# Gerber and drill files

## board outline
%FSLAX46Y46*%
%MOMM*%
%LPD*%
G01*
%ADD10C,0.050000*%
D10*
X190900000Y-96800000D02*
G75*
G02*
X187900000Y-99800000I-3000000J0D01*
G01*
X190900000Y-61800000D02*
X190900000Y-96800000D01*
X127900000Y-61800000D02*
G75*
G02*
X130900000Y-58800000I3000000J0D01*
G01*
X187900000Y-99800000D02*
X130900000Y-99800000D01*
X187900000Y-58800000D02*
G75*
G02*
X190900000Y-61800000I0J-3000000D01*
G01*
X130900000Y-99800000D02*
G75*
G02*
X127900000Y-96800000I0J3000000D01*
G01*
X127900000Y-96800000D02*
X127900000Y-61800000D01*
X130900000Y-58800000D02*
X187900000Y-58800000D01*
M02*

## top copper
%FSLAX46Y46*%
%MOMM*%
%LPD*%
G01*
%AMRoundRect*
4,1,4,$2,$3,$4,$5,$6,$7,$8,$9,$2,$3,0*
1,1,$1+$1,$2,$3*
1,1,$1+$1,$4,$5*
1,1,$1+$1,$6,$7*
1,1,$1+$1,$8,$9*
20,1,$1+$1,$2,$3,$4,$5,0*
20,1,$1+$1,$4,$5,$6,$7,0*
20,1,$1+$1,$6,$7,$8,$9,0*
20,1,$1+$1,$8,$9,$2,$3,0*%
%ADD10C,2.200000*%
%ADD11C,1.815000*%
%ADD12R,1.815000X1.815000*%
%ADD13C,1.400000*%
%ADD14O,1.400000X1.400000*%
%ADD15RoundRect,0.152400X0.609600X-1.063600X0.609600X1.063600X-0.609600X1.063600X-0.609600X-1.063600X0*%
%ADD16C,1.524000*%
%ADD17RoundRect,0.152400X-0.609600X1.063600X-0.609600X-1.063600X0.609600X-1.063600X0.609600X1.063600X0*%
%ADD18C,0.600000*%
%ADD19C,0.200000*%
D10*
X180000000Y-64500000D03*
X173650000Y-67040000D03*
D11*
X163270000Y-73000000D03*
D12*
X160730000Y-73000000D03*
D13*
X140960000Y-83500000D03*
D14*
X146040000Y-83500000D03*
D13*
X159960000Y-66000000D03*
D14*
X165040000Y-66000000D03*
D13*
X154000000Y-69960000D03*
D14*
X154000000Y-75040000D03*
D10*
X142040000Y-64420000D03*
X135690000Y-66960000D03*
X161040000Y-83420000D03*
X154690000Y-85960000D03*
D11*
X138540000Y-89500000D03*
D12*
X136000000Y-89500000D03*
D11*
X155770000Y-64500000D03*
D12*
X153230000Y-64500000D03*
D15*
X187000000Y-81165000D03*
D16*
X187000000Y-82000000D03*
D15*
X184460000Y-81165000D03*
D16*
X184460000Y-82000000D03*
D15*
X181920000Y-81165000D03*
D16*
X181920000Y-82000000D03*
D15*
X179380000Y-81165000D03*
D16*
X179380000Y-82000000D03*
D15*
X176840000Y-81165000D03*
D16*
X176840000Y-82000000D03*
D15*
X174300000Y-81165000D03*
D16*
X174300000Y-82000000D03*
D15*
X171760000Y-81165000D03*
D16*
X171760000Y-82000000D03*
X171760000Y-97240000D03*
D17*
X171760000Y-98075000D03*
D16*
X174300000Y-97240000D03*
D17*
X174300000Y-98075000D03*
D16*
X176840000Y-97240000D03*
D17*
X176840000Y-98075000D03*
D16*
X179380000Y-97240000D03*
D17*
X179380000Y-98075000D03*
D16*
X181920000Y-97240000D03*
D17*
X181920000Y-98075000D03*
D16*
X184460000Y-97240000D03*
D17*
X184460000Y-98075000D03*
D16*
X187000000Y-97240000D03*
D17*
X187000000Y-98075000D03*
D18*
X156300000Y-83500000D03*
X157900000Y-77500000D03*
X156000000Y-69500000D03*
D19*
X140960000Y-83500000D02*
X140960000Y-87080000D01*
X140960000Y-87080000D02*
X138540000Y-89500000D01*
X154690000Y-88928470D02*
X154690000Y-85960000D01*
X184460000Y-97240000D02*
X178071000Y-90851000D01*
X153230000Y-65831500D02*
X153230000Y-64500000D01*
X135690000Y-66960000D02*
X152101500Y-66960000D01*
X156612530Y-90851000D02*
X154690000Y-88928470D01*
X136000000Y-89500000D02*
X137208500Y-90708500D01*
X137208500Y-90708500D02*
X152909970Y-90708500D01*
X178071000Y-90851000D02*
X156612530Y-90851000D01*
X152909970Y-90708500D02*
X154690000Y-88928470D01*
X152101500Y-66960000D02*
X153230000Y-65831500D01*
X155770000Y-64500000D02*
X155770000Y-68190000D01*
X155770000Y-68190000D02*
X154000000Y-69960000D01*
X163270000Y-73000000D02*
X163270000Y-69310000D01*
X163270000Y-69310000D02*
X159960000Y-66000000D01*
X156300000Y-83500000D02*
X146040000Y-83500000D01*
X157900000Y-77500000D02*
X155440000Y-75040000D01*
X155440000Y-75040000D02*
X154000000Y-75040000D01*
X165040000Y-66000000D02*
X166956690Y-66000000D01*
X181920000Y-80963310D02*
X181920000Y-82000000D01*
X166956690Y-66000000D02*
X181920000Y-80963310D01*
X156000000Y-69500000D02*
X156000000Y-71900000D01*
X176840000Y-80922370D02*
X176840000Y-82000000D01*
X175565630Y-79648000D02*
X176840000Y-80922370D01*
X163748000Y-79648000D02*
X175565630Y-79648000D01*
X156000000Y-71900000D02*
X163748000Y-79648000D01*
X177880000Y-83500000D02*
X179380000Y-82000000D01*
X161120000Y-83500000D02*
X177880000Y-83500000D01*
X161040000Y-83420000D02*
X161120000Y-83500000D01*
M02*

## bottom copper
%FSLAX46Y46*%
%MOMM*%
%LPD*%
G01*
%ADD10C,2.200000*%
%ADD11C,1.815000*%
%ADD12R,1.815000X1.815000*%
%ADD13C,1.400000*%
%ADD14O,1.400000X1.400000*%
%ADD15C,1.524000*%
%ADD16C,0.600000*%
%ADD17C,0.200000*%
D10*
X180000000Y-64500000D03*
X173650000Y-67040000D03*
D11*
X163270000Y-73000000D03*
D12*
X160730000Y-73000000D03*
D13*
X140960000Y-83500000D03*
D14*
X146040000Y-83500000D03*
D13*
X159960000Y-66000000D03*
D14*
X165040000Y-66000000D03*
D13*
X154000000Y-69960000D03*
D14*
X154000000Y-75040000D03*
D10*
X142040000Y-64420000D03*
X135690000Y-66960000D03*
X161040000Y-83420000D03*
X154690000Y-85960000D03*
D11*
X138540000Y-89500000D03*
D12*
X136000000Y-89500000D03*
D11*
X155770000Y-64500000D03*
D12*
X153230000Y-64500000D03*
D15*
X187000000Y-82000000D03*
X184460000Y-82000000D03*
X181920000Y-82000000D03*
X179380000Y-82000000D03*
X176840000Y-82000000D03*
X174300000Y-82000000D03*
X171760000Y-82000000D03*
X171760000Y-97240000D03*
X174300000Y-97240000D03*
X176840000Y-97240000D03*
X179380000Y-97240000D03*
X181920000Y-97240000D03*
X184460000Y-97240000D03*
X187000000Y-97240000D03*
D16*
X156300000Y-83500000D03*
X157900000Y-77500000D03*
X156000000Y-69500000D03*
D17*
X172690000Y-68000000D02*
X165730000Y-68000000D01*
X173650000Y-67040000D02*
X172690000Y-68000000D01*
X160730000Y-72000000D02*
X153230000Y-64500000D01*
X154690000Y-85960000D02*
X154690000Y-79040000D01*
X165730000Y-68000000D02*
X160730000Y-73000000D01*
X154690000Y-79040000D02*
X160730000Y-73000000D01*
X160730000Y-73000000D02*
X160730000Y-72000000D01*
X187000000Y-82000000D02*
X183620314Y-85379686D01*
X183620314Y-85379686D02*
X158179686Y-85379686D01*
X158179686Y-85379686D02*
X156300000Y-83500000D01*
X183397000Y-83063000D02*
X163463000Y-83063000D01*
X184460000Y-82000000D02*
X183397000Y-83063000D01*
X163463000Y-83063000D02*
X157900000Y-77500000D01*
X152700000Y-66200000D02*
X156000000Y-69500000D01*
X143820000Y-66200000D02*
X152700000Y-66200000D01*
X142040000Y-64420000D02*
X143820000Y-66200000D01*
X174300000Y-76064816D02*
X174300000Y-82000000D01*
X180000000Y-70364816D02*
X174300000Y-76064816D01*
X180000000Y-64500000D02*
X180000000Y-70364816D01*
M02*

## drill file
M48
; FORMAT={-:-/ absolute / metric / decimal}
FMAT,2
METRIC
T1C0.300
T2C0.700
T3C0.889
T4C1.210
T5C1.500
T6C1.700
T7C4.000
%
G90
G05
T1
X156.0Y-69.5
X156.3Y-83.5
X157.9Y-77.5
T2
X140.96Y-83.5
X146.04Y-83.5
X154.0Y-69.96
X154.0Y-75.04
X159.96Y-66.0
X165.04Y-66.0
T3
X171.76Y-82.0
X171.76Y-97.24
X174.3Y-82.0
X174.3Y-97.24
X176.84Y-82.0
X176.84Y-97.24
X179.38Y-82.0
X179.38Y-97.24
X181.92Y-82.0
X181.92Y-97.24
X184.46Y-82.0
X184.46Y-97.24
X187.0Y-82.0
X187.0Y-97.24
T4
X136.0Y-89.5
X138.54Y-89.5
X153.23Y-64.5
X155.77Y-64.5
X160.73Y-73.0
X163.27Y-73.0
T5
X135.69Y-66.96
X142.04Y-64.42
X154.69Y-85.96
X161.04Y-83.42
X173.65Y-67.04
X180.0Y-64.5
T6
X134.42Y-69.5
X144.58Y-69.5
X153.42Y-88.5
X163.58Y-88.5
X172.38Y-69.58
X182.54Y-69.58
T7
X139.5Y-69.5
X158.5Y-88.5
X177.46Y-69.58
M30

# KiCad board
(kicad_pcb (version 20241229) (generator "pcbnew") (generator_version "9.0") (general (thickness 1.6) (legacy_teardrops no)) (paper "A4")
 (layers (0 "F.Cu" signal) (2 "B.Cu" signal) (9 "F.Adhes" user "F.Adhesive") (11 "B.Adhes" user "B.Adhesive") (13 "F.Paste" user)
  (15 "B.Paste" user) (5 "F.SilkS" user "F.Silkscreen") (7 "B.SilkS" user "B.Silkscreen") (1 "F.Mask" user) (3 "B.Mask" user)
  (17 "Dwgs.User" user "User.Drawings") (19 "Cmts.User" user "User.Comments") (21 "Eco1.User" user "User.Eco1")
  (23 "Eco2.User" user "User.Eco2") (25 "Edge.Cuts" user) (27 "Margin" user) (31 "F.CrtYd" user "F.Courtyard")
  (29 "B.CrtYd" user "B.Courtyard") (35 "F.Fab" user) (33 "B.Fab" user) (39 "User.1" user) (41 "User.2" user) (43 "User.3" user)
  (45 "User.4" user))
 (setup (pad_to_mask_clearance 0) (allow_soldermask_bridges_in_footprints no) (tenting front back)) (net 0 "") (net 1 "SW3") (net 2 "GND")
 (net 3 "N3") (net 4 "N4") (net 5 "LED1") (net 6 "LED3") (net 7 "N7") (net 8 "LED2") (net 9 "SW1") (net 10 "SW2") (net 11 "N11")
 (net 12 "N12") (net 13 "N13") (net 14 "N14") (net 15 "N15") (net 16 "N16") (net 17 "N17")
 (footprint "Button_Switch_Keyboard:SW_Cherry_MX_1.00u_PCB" (layer "F.Cu") (at 180 64.5)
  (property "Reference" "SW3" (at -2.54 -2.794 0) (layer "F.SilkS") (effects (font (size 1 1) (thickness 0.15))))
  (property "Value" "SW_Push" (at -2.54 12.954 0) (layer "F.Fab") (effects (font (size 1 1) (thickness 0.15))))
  (pad "" np_thru_hole circle (at -7.62 5.08) (size 1.7 1.7) (drill 1.7) (layers "*.Cu" "*.Mask"))
  (pad "" np_thru_hole circle (at -2.54 5.08) (size 4 4) (drill 4) (layers "*.Cu" "*.Mask"))
  (pad "" np_thru_hole circle (at 2.54 5.08) (size 1.7 1.7) (drill 1.7) (layers "*.Cu" "*.Mask"))
  (pad "1" thru_hole circle (at 0 0) (size 2.2 2.2) (drill 1.5) (layers "*.Cu" "*.Mask") (remove_unused_layers no) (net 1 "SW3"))
  (pad "2" thru_hole circle (at -6.35 2.54) (size 2.2 2.2) (drill 1.5) (layers "*.Cu" "*.Mask") (remove_unused_layers no) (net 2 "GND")))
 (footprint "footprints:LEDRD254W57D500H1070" (layer "F.Cu") (at 162 73)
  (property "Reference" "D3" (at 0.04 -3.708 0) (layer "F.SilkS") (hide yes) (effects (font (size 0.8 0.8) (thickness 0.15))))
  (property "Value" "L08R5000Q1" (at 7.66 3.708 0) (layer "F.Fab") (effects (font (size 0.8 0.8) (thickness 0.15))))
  (pad "A" thru_hole circle (at 1.27 0) (size 1.815 1.815) (drill 1.21) (layers "*.Cu" "*.Mask") (remove_unused_layers no) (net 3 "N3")
   (solder_mask_margin 0.102))
  (pad "C" thru_hole rect (at -1.27 0) (size 1.815 1.815) (drill 1.21) (layers "*.Cu" "*.Mask") (remove_unused_layers no) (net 2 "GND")
   (solder_mask_margin 0.102)))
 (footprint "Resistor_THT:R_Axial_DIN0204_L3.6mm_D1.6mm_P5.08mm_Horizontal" (layer "F.Cu") (at 140.96 83.5)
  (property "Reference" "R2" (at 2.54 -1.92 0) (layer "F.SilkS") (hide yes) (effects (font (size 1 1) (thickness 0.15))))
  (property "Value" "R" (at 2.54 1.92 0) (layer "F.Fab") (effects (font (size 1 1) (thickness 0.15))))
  (pad "1" thru_hole circle (at 0 0) (size 1.4 1.4) (drill 0.7) (layers "*.Cu" "*.Mask") (remove_unused_layers no) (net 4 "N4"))
  (pad "2" thru_hole oval (at 5.08 0) (size 1.4 1.4) (drill 0.7) (layers "*.Cu" "*.Mask") (remove_unused_layers no) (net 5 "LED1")))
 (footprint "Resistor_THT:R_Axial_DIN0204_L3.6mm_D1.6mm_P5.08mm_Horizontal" (layer "F.Cu") (at 159.96 66)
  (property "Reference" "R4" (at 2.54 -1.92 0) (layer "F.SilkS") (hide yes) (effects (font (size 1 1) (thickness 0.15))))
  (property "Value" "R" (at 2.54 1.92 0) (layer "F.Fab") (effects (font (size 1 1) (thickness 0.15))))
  (pad "1" thru_hole circle (at 0 0) (size 1.4 1.4) (drill 0.7) (layers "*.Cu" "*.Mask") (remove_unused_layers no) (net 3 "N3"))
  (pad "2" thru_hole oval (at 5.08 0) (size 1.4 1.4) (drill 0.7) (layers "*.Cu" "*.Mask") (remove_unused_layers no) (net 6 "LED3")))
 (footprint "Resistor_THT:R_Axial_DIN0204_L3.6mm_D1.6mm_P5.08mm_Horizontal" (layer "F.Cu") (at 154 69.96 -90)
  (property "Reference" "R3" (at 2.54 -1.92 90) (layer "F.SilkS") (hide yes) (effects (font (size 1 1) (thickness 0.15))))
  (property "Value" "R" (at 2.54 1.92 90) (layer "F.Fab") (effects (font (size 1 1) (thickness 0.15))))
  (pad "1" thru_hole circle (at 0 0 270) (size 1.4 1.4) (drill 0.7) (layers "*.Cu" "*.Mask") (remove_unused_layers no) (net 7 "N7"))
  (pad "2" thru_hole oval (at 5.08 0 270) (size 1.4 1.4) (drill 0.7) (layers "*.Cu" "*.Mask") (remove_unused_layers no) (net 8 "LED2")))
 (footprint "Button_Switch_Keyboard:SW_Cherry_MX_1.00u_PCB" (layer "F.Cu") (at 142.04 64.42)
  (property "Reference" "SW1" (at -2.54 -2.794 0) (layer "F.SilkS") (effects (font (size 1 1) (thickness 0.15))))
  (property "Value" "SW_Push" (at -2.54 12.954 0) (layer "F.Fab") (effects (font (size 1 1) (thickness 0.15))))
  (pad "" np_thru_hole circle (at -7.62 5.08) (size 1.7 1.7) (drill 1.7) (layers "*.Cu" "*.Mask"))
  (pad "" np_thru_hole circle (at -2.54 5.08) (size 4 4) (drill 4) (layers "*.Cu" "*.Mask"))
  (pad "" np_thru_hole circle (at 2.54 5.08) (size 1.7 1.7) (drill 1.7) (layers "*.Cu" "*.Mask"))
  (pad "1" thru_hole circle (at 0 0) (size 2.2 2.2) (drill 1.5) (layers "*.Cu" "*.Mask") (remove_unused_layers no) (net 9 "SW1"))
  (pad "2" thru_hole circle (at -6.35 2.54) (size 2.2 2.2) (drill 1.5) (layers "*.Cu" "*.Mask") (remove_unused_layers no) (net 2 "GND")))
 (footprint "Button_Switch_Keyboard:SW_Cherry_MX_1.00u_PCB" (layer "F.Cu") (at 161.04 83.42)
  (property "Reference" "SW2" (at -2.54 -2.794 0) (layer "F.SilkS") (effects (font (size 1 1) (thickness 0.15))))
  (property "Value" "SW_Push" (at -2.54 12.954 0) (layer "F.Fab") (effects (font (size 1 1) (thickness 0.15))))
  (pad "" np_thru_hole circle (at -7.62 5.08) (size 1.7 1.7) (drill 1.7) (layers "*.Cu" "*.Mask"))
  (pad "" np_thru_hole circle (at -2.54 5.08) (size 4 4) (drill 4) (layers "*.Cu" "*.Mask"))
  (pad "" np_thru_hole circle (at 2.54 5.08) (size 1.7 1.7) (drill 1.7) (layers "*.Cu" "*.Mask"))
  (pad "1" thru_hole circle (at 0 0) (size 2.2 2.2) (drill 1.5) (layers "*.Cu" "*.Mask") (remove_unused_layers no) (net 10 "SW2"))
  (pad "2" thru_hole circle (at -6.35 2.54) (size 2.2 2.2) (drill 1.5) (layers "*.Cu" "*.Mask") (remove_unused_layers no) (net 2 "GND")))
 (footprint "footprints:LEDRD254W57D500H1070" (layer "F.Cu") (at 137.27 89.5)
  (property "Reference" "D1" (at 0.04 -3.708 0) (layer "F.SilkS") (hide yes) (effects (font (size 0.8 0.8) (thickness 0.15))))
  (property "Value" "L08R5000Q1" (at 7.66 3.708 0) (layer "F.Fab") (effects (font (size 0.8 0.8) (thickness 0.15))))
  (pad "A" thru_hole circle (at 1.27 0) (size 1.815 1.815) (drill 1.21) (layers "*.Cu" "*.Mask") (remove_unused_layers no) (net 4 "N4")
   (solder_mask_margin 0.102))
  (pad "C" thru_hole rect (at -1.27 0) (size 1.815 1.815) (drill 1.21) (layers "*.Cu" "*.Mask") (remove_unused_layers no) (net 2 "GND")
   (solder_mask_margin 0.102)))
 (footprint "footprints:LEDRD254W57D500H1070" (layer "F.Cu") (at 154.5 64.5)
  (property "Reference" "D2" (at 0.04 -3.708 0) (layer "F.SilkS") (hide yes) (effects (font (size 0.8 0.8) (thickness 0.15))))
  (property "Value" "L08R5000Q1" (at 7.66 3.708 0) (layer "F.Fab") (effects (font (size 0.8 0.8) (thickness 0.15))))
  (pad "A" thru_hole circle (at 1.27 0) (size 1.815 1.815) (drill 1.21) (layers "*.Cu" "*.Mask") (remove_unused_layers no) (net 7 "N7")
   (solder_mask_margin 0.102))
  (pad "C" thru_hole rect (at -1.27 0) (size 1.815 1.815) (drill 1.21) (layers "*.Cu" "*.Mask") (remove_unused_layers no) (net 2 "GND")
   (solder_mask_margin 0.102)))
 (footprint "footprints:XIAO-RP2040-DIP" (layer "F.Cu") (at 179.38 89.62 -90)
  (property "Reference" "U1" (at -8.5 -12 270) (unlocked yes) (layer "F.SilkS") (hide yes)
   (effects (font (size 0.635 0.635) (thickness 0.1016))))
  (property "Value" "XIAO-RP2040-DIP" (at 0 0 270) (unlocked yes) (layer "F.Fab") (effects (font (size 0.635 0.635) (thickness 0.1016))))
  (pad "1" smd roundrect (at -8.455 -7.62 90) (size 2.432 1.524) (layers "F.Cu" "F.Mask") (roundrect_rratio 0.1) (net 5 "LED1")
   (thermal_bridge_angle 45))
  (pad "1" thru_hole circle (at -7.62 -7.62 90) (size 1.524 1.524) (drill 0.889) (layers "*.Cu" "*.Mask") (remove_unused_layers no)
   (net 5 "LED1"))
  (pad "2" smd roundrect (at -8.455 -5.08 90) (size 2.432 1.524) (layers "F.Cu" "F.Mask") (roundrect_rratio 0.1) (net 8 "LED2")
   (thermal_bridge_angle 45))
  (pad "2" thru_hole circle (at -7.62 -5.08 90) (size 1.524 1.524) (drill 0.889) (layers "*.Cu" "*.Mask") (remove_unused_layers no)
   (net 8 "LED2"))
  (pad "3" smd roundrect (at -8.455 -2.54 90) (size 2.432 1.524) (layers "F.Cu" "F.Mask") (roundrect_rratio 0.1) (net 6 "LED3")
   (thermal_bridge_angle 45))
  (pad "3" thru_hole circle (at -7.62 -2.54 90) (size 1.524 1.524) (drill 0.889) (layers "*.Cu" "*.Mask") (remove_unused_layers no)
   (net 6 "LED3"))
  (pad "4" smd roundrect (at -8.455 0 90) (size 2.432 1.524) (layers "F.Cu" "F.Mask") (roundrect_rratio 0.1) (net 10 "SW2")
   (thermal_bridge_angle 45))
  (pad "4" thru_hole circle (at -7.62 0 90) (size 1.524 1.524) (drill 0.889) (layers "*.Cu" "*.Mask") (remove_unused_layers no)
   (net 10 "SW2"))
  (pad "5" smd roundrect (at -8.455 2.54 90) (size 2.432 1.524) (layers "F.Cu" "F.Mask") (roundrect_rratio 0.1) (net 9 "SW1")
   (thermal_bridge_angle 45))
  (pad "5" thru_hole circle (at -7.62 2.54 90) (size 1.524 1.524) (drill 0.889) (layers "*.Cu" "*.Mask") (remove_unused_layers no)
   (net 9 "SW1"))
  (pad "6" smd roundrect (at -8.455 5.08 90) (size 2.432 1.524) (layers "F.Cu" "F.Mask") (roundrect_rratio 0.1) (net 1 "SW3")
   (thermal_bridge_angle 45))
  (pad "6" thru_hole circle (at -7.62 5.08 90) (size 1.524 1.524) (drill 0.889) (layers "*.Cu" "*.Mask") (remove_unused_layers no)
   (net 1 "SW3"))
  (pad "7" smd roundrect (at -8.455 7.62 90) (size 2.432 1.524) (layers "F.Cu" "F.Mask") (roundrect_rratio 0.1) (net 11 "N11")
   (thermal_bridge_angle 45))
  (pad "7" thru_hole circle (at -7.62 7.62 90) (size 1.524 1.524) (drill 0.889) (layers "*.Cu" "*.Mask") (remove_unused_layers no)
   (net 11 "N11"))
  (pad "8" thru_hole circle (at 7.62 7.62 270) (size 1.524 1.524) (drill 0.889) (layers "*.Cu" "*.Mask") (remove_unused_layers no)
   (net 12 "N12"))
  (pad "8" smd roundrect (at 8.455 7.62 270) (size 2.432 1.524) (layers "F.Cu" "F.Mask") (roundrect_rratio 0.1) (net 12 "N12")
   (thermal_bridge_angle 45))
  (pad "9" thru_hole circle (at 7.62 5.08 270) (size 1.524 1.524) (drill 0.889) (layers "*.Cu" "*.Mask") (remove_unused_layers no)
   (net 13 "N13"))
  (pad "9" smd roundrect (at 8.455 5.08 270) (size 2.432 1.524) (layers "F.Cu" "F.Mask") (roundrect_rratio 0.1) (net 13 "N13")
   (thermal_bridge_angle 45))
  (pad "10" thru_hole circle (at 7.62 2.54 270) (size 1.524 1.524) (drill 0.889) (layers "*.Cu" "*.Mask") (remove_unused_layers no)
   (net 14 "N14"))
  (pad "10" smd roundrect (at 8.455 2.54 270) (size 2.432 1.524) (layers "F.Cu" "F.Mask") (roundrect_rratio 0.1) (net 14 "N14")
   (thermal_bridge_angle 45))
  (pad "11" thru_hole circle (at 7.62 0 270) (size 1.524 1.524) (drill 0.889) (layers "*.Cu" "*.Mask") (remove_unused_layers no)
   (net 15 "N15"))
  (pad "11" smd roundrect (at 8.455 0 270) (size 2.432 1.524) (layers "F.Cu" "F.Mask") (roundrect_rratio 0.1) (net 15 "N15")
   (thermal_bridge_angle 45))
  (pad "12" thru_hole circle (at 7.62 -2.54 270) (size 1.524 1.524) (drill 0.889) (layers "*.Cu" "*.Mask") (remove_unused_layers no)
   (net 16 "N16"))
  (pad "12" smd roundrect (at 8.455 -2.54 270) (size 2.432 1.524) (layers "F.Cu" "F.Mask") (roundrect_rratio 0.1) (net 16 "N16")
   (thermal_bridge_angle 45))
  (pad "13" thru_hole circle (at 7.62 -5.08 270) (size 1.524 1.524) (drill 0.889) (layers "*.Cu" "*.Mask") (remove_unused_layers no)
   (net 2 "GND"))
  (pad "13" smd roundrect (at 8.455 -5.08 270) (size 2.432 1.524) (layers "F.Cu" "F.Mask") (roundrect_rratio 0.1) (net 2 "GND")
   (thermal_bridge_angle 45))
  (pad "14" thru_hole circle (at 7.62 -7.62 270) (size 1.524 1.524) (drill 0.889) (layers "*.Cu" "*.Mask") (remove_unused_layers no)
   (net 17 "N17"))
  (pad "14" smd roundrect (at 8.455 -7.62 270) (size 2.432 1.524) (layers "F.Cu" "F.Mask") (roundrect_rratio 0.1) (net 17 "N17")
   (thermal_bridge_angle 45)))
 (gr_arc (start 190.9 96.8) (mid 190.02132 98.92132) (end 187.9 99.8) (stroke (width 0.05) (type default)) (layer "Edge.Cuts"))
 (gr_line (start 190.9 61.8) (end 190.9 96.8) (stroke (width 0.05) (type default)) (layer "Edge.Cuts"))
 (gr_arc (start 127.9 61.8) (mid 128.77868 59.67868) (end 130.9 58.8) (stroke (width 0.05) (type default)) (layer "Edge.Cuts"))
 (gr_line (start 187.9 99.8) (end 130.9 99.8) (stroke (width 0.05) (type default)) (layer "Edge.Cuts"))
 (gr_arc (start 187.9 58.8) (mid 190.02132 59.67868) (end 190.9 61.8) (stroke (width 0.05) (type default)) (layer "Edge.Cuts"))
 (gr_arc (start 130.9 99.8) (mid 128.77868 98.92132) (end 127.9 96.8) (stroke (width 0.05) (type default)) (layer "Edge.Cuts"))
 (gr_line (start 127.9 96.8) (end 127.9 61.8) (stroke (width 0.05) (type default)) (layer "Edge.Cuts"))
 (gr_line (start 130.9 58.8) (end 187.9 58.8) (stroke (width 0.05) (type default)) (layer "Edge.Cuts"))
 (segment (start 140.96 83.5) (end 140.96 87.08) (width 0.2) (layer "F.Cu") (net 4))
 (segment (start 140.96 87.08) (end 138.54 89.5) (width 0.2) (layer "F.Cu") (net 4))
 (segment (start 154.69 88.92847) (end 154.69 85.96) (width 0.2) (layer "F.Cu") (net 2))
 (segment (start 184.46 97.24) (end 178.071 90.851) (width 0.2) (layer "F.Cu") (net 2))
 (segment (start 153.23 65.8315) (end 153.23 64.5) (width 0.2) (layer "F.Cu") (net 2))
 (segment (start 135.69 66.96) (end 152.1015 66.96) (width 0.2) (layer "F.Cu") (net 2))
 (segment (start 156.61253 90.851) (end 154.69 88.92847) (width 0.2) (layer "F.Cu") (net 2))
 (segment (start 136 89.5) (end 137.2085 90.7085) (width 0.2) (layer "F.Cu") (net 2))
 (segment (start 137.2085 90.7085) (end 152.90997 90.7085) (width 0.2) (layer "F.Cu") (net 2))
 (segment (start 178.071 90.851) (end 156.61253 90.851) (width 0.2) (layer "F.Cu") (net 2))
 (segment (start 152.90997 90.7085) (end 154.69 88.92847) (width 0.2) (layer "F.Cu") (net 2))
 (segment (start 152.1015 66.96) (end 153.23 65.8315) (width 0.2) (layer "F.Cu") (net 2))
 (segment (start 172.69 68) (end 165.73 68) (width 0.2) (layer "B.Cu") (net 2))
 (segment (start 173.65 67.04) (end 172.69 68) (width 0.2) (layer "B.Cu") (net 2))
 (segment (start 160.73 72) (end 153.23 64.5) (width 0.2) (layer "B.Cu") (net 2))
 (segment (start 154.69 85.96) (end 154.69 79.04) (width 0.2) (layer "B.Cu") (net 2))
 (segment (start 165.73 68) (end 160.73 73) (width 0.2) (layer "B.Cu") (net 2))
 (segment (start 154.69 79.04) (end 160.73 73) (width 0.2) (layer "B.Cu") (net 2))
 (segment (start 160.73 73) (end 160.73 72) (width 0.2) (layer "B.Cu") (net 2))
 (segment (start 155.77 64.5) (end 155.77 68.19) (width 0.2) (layer "F.Cu") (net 7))
 (segment (start 155.77 68.19) (end 154 69.96) (width 0.2) (layer "F.Cu") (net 7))
 (segment (start 163.27 73) (end 163.27 69.31) (width 0.2) (layer "F.Cu") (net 3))
 (segment (start 163.27 69.31) (end 159.96 66) (width 0.2) (layer "F.Cu") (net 3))
 (segment (start 156.3 83.5) (end 146.04 83.5) (width 0.2) (layer "F.Cu") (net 5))
 (via (at 156.3 83.5) (size 0.6) (drill 0.3) (layers "F.Cu" "B.Cu") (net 5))
 (segment (start 187 82) (end 183.620314 85.379686) (width 0.2) (layer "B.Cu") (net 5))
 (segment (start 183.620314 85.379686) (end 158.179686 85.379686) (width 0.2) (layer "B.Cu") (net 5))
 (segment (start 158.179686 85.379686) (end 156.3 83.5) (width 0.2) (layer "B.Cu") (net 5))
 (segment (start 157.9 77.5) (end 155.44 75.04) (width 0.2) (layer "F.Cu") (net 8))
 (segment (start 155.44 75.04) (end 154 75.04) (width 0.2) (layer "F.Cu") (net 8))
 (via (at 157.9 77.5) (size 0.6) (drill 0.3) (layers "F.Cu" "B.Cu") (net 8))
 (segment (start 183.397 83.063) (end 163.463 83.063) (width 0.2) (layer "B.Cu") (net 8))
 (segment (start 184.46 82) (end 183.397 83.063) (width 0.2) (layer "B.Cu") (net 8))
 (segment (start 163.463 83.063) (end 157.9 77.5) (width 0.2) (layer "B.Cu") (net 8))
 (segment (start 165.04 66) (end 166.95669 66) (width 0.2) (layer "F.Cu") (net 6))
 (segment (start 181.92 80.96331) (end 181.92 82) (width 0.2) (layer "F.Cu") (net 6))
 (segment (start 166.95669 66) (end 181.92 80.96331) (width 0.2) (layer "F.Cu") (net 6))
 (segment (start 156 69.5) (end 156 71.9) (width 0.2) (layer "F.Cu") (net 9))
 (segment (start 176.84 80.92237) (end 176.84 82) (width 0.2) (layer "F.Cu") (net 9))
 (segment (start 175.56563 79.648) (end 176.84 80.92237) (width 0.2) (layer "F.Cu") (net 9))
 (segment (start 163.748 79.648) (end 175.56563 79.648) (width 0.2) (layer "F.Cu") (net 9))
 (segment (start 156 71.9) (end 163.748 79.648) (width 0.2) (layer "F.Cu") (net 9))
 (via (at 156 69.5) (size 0.6) (drill 0.3) (layers "F.Cu" "B.Cu") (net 9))
 (segment (start 152.7 66.2) (end 156 69.5) (width 0.2) (layer "B.Cu") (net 9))
 (segment (start 143.82 66.2) (end 152.7 66.2) (width 0.2) (layer "B.Cu") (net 9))
 (segment (start 142.04 64.42) (end 143.82 66.2) (width 0.2) (layer "B.Cu") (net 9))
 (segment (start 177.88 83.5) (end 179.38 82) (width 0.2) (layer "F.Cu") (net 10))
 (segment (start 161.12 83.5) (end 177.88 83.5) (width 0.2) (layer "F.Cu") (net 10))
 (segment (start 161.04 83.42) (end 161.12 83.5) (width 0.2) (layer "F.Cu") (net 10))
 (segment (start 174.3 76.064816) (end 174.3 82) (width 0.2) (layer "B.Cu") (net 1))
 (segment (start 180 70.364816) (end 174.3 76.064816) (width 0.2) (layer "B.Cu") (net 1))
 (segment (start 180 64.5) (end 180 70.364816) (width 0.2) (layer "B.Cu") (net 1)))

